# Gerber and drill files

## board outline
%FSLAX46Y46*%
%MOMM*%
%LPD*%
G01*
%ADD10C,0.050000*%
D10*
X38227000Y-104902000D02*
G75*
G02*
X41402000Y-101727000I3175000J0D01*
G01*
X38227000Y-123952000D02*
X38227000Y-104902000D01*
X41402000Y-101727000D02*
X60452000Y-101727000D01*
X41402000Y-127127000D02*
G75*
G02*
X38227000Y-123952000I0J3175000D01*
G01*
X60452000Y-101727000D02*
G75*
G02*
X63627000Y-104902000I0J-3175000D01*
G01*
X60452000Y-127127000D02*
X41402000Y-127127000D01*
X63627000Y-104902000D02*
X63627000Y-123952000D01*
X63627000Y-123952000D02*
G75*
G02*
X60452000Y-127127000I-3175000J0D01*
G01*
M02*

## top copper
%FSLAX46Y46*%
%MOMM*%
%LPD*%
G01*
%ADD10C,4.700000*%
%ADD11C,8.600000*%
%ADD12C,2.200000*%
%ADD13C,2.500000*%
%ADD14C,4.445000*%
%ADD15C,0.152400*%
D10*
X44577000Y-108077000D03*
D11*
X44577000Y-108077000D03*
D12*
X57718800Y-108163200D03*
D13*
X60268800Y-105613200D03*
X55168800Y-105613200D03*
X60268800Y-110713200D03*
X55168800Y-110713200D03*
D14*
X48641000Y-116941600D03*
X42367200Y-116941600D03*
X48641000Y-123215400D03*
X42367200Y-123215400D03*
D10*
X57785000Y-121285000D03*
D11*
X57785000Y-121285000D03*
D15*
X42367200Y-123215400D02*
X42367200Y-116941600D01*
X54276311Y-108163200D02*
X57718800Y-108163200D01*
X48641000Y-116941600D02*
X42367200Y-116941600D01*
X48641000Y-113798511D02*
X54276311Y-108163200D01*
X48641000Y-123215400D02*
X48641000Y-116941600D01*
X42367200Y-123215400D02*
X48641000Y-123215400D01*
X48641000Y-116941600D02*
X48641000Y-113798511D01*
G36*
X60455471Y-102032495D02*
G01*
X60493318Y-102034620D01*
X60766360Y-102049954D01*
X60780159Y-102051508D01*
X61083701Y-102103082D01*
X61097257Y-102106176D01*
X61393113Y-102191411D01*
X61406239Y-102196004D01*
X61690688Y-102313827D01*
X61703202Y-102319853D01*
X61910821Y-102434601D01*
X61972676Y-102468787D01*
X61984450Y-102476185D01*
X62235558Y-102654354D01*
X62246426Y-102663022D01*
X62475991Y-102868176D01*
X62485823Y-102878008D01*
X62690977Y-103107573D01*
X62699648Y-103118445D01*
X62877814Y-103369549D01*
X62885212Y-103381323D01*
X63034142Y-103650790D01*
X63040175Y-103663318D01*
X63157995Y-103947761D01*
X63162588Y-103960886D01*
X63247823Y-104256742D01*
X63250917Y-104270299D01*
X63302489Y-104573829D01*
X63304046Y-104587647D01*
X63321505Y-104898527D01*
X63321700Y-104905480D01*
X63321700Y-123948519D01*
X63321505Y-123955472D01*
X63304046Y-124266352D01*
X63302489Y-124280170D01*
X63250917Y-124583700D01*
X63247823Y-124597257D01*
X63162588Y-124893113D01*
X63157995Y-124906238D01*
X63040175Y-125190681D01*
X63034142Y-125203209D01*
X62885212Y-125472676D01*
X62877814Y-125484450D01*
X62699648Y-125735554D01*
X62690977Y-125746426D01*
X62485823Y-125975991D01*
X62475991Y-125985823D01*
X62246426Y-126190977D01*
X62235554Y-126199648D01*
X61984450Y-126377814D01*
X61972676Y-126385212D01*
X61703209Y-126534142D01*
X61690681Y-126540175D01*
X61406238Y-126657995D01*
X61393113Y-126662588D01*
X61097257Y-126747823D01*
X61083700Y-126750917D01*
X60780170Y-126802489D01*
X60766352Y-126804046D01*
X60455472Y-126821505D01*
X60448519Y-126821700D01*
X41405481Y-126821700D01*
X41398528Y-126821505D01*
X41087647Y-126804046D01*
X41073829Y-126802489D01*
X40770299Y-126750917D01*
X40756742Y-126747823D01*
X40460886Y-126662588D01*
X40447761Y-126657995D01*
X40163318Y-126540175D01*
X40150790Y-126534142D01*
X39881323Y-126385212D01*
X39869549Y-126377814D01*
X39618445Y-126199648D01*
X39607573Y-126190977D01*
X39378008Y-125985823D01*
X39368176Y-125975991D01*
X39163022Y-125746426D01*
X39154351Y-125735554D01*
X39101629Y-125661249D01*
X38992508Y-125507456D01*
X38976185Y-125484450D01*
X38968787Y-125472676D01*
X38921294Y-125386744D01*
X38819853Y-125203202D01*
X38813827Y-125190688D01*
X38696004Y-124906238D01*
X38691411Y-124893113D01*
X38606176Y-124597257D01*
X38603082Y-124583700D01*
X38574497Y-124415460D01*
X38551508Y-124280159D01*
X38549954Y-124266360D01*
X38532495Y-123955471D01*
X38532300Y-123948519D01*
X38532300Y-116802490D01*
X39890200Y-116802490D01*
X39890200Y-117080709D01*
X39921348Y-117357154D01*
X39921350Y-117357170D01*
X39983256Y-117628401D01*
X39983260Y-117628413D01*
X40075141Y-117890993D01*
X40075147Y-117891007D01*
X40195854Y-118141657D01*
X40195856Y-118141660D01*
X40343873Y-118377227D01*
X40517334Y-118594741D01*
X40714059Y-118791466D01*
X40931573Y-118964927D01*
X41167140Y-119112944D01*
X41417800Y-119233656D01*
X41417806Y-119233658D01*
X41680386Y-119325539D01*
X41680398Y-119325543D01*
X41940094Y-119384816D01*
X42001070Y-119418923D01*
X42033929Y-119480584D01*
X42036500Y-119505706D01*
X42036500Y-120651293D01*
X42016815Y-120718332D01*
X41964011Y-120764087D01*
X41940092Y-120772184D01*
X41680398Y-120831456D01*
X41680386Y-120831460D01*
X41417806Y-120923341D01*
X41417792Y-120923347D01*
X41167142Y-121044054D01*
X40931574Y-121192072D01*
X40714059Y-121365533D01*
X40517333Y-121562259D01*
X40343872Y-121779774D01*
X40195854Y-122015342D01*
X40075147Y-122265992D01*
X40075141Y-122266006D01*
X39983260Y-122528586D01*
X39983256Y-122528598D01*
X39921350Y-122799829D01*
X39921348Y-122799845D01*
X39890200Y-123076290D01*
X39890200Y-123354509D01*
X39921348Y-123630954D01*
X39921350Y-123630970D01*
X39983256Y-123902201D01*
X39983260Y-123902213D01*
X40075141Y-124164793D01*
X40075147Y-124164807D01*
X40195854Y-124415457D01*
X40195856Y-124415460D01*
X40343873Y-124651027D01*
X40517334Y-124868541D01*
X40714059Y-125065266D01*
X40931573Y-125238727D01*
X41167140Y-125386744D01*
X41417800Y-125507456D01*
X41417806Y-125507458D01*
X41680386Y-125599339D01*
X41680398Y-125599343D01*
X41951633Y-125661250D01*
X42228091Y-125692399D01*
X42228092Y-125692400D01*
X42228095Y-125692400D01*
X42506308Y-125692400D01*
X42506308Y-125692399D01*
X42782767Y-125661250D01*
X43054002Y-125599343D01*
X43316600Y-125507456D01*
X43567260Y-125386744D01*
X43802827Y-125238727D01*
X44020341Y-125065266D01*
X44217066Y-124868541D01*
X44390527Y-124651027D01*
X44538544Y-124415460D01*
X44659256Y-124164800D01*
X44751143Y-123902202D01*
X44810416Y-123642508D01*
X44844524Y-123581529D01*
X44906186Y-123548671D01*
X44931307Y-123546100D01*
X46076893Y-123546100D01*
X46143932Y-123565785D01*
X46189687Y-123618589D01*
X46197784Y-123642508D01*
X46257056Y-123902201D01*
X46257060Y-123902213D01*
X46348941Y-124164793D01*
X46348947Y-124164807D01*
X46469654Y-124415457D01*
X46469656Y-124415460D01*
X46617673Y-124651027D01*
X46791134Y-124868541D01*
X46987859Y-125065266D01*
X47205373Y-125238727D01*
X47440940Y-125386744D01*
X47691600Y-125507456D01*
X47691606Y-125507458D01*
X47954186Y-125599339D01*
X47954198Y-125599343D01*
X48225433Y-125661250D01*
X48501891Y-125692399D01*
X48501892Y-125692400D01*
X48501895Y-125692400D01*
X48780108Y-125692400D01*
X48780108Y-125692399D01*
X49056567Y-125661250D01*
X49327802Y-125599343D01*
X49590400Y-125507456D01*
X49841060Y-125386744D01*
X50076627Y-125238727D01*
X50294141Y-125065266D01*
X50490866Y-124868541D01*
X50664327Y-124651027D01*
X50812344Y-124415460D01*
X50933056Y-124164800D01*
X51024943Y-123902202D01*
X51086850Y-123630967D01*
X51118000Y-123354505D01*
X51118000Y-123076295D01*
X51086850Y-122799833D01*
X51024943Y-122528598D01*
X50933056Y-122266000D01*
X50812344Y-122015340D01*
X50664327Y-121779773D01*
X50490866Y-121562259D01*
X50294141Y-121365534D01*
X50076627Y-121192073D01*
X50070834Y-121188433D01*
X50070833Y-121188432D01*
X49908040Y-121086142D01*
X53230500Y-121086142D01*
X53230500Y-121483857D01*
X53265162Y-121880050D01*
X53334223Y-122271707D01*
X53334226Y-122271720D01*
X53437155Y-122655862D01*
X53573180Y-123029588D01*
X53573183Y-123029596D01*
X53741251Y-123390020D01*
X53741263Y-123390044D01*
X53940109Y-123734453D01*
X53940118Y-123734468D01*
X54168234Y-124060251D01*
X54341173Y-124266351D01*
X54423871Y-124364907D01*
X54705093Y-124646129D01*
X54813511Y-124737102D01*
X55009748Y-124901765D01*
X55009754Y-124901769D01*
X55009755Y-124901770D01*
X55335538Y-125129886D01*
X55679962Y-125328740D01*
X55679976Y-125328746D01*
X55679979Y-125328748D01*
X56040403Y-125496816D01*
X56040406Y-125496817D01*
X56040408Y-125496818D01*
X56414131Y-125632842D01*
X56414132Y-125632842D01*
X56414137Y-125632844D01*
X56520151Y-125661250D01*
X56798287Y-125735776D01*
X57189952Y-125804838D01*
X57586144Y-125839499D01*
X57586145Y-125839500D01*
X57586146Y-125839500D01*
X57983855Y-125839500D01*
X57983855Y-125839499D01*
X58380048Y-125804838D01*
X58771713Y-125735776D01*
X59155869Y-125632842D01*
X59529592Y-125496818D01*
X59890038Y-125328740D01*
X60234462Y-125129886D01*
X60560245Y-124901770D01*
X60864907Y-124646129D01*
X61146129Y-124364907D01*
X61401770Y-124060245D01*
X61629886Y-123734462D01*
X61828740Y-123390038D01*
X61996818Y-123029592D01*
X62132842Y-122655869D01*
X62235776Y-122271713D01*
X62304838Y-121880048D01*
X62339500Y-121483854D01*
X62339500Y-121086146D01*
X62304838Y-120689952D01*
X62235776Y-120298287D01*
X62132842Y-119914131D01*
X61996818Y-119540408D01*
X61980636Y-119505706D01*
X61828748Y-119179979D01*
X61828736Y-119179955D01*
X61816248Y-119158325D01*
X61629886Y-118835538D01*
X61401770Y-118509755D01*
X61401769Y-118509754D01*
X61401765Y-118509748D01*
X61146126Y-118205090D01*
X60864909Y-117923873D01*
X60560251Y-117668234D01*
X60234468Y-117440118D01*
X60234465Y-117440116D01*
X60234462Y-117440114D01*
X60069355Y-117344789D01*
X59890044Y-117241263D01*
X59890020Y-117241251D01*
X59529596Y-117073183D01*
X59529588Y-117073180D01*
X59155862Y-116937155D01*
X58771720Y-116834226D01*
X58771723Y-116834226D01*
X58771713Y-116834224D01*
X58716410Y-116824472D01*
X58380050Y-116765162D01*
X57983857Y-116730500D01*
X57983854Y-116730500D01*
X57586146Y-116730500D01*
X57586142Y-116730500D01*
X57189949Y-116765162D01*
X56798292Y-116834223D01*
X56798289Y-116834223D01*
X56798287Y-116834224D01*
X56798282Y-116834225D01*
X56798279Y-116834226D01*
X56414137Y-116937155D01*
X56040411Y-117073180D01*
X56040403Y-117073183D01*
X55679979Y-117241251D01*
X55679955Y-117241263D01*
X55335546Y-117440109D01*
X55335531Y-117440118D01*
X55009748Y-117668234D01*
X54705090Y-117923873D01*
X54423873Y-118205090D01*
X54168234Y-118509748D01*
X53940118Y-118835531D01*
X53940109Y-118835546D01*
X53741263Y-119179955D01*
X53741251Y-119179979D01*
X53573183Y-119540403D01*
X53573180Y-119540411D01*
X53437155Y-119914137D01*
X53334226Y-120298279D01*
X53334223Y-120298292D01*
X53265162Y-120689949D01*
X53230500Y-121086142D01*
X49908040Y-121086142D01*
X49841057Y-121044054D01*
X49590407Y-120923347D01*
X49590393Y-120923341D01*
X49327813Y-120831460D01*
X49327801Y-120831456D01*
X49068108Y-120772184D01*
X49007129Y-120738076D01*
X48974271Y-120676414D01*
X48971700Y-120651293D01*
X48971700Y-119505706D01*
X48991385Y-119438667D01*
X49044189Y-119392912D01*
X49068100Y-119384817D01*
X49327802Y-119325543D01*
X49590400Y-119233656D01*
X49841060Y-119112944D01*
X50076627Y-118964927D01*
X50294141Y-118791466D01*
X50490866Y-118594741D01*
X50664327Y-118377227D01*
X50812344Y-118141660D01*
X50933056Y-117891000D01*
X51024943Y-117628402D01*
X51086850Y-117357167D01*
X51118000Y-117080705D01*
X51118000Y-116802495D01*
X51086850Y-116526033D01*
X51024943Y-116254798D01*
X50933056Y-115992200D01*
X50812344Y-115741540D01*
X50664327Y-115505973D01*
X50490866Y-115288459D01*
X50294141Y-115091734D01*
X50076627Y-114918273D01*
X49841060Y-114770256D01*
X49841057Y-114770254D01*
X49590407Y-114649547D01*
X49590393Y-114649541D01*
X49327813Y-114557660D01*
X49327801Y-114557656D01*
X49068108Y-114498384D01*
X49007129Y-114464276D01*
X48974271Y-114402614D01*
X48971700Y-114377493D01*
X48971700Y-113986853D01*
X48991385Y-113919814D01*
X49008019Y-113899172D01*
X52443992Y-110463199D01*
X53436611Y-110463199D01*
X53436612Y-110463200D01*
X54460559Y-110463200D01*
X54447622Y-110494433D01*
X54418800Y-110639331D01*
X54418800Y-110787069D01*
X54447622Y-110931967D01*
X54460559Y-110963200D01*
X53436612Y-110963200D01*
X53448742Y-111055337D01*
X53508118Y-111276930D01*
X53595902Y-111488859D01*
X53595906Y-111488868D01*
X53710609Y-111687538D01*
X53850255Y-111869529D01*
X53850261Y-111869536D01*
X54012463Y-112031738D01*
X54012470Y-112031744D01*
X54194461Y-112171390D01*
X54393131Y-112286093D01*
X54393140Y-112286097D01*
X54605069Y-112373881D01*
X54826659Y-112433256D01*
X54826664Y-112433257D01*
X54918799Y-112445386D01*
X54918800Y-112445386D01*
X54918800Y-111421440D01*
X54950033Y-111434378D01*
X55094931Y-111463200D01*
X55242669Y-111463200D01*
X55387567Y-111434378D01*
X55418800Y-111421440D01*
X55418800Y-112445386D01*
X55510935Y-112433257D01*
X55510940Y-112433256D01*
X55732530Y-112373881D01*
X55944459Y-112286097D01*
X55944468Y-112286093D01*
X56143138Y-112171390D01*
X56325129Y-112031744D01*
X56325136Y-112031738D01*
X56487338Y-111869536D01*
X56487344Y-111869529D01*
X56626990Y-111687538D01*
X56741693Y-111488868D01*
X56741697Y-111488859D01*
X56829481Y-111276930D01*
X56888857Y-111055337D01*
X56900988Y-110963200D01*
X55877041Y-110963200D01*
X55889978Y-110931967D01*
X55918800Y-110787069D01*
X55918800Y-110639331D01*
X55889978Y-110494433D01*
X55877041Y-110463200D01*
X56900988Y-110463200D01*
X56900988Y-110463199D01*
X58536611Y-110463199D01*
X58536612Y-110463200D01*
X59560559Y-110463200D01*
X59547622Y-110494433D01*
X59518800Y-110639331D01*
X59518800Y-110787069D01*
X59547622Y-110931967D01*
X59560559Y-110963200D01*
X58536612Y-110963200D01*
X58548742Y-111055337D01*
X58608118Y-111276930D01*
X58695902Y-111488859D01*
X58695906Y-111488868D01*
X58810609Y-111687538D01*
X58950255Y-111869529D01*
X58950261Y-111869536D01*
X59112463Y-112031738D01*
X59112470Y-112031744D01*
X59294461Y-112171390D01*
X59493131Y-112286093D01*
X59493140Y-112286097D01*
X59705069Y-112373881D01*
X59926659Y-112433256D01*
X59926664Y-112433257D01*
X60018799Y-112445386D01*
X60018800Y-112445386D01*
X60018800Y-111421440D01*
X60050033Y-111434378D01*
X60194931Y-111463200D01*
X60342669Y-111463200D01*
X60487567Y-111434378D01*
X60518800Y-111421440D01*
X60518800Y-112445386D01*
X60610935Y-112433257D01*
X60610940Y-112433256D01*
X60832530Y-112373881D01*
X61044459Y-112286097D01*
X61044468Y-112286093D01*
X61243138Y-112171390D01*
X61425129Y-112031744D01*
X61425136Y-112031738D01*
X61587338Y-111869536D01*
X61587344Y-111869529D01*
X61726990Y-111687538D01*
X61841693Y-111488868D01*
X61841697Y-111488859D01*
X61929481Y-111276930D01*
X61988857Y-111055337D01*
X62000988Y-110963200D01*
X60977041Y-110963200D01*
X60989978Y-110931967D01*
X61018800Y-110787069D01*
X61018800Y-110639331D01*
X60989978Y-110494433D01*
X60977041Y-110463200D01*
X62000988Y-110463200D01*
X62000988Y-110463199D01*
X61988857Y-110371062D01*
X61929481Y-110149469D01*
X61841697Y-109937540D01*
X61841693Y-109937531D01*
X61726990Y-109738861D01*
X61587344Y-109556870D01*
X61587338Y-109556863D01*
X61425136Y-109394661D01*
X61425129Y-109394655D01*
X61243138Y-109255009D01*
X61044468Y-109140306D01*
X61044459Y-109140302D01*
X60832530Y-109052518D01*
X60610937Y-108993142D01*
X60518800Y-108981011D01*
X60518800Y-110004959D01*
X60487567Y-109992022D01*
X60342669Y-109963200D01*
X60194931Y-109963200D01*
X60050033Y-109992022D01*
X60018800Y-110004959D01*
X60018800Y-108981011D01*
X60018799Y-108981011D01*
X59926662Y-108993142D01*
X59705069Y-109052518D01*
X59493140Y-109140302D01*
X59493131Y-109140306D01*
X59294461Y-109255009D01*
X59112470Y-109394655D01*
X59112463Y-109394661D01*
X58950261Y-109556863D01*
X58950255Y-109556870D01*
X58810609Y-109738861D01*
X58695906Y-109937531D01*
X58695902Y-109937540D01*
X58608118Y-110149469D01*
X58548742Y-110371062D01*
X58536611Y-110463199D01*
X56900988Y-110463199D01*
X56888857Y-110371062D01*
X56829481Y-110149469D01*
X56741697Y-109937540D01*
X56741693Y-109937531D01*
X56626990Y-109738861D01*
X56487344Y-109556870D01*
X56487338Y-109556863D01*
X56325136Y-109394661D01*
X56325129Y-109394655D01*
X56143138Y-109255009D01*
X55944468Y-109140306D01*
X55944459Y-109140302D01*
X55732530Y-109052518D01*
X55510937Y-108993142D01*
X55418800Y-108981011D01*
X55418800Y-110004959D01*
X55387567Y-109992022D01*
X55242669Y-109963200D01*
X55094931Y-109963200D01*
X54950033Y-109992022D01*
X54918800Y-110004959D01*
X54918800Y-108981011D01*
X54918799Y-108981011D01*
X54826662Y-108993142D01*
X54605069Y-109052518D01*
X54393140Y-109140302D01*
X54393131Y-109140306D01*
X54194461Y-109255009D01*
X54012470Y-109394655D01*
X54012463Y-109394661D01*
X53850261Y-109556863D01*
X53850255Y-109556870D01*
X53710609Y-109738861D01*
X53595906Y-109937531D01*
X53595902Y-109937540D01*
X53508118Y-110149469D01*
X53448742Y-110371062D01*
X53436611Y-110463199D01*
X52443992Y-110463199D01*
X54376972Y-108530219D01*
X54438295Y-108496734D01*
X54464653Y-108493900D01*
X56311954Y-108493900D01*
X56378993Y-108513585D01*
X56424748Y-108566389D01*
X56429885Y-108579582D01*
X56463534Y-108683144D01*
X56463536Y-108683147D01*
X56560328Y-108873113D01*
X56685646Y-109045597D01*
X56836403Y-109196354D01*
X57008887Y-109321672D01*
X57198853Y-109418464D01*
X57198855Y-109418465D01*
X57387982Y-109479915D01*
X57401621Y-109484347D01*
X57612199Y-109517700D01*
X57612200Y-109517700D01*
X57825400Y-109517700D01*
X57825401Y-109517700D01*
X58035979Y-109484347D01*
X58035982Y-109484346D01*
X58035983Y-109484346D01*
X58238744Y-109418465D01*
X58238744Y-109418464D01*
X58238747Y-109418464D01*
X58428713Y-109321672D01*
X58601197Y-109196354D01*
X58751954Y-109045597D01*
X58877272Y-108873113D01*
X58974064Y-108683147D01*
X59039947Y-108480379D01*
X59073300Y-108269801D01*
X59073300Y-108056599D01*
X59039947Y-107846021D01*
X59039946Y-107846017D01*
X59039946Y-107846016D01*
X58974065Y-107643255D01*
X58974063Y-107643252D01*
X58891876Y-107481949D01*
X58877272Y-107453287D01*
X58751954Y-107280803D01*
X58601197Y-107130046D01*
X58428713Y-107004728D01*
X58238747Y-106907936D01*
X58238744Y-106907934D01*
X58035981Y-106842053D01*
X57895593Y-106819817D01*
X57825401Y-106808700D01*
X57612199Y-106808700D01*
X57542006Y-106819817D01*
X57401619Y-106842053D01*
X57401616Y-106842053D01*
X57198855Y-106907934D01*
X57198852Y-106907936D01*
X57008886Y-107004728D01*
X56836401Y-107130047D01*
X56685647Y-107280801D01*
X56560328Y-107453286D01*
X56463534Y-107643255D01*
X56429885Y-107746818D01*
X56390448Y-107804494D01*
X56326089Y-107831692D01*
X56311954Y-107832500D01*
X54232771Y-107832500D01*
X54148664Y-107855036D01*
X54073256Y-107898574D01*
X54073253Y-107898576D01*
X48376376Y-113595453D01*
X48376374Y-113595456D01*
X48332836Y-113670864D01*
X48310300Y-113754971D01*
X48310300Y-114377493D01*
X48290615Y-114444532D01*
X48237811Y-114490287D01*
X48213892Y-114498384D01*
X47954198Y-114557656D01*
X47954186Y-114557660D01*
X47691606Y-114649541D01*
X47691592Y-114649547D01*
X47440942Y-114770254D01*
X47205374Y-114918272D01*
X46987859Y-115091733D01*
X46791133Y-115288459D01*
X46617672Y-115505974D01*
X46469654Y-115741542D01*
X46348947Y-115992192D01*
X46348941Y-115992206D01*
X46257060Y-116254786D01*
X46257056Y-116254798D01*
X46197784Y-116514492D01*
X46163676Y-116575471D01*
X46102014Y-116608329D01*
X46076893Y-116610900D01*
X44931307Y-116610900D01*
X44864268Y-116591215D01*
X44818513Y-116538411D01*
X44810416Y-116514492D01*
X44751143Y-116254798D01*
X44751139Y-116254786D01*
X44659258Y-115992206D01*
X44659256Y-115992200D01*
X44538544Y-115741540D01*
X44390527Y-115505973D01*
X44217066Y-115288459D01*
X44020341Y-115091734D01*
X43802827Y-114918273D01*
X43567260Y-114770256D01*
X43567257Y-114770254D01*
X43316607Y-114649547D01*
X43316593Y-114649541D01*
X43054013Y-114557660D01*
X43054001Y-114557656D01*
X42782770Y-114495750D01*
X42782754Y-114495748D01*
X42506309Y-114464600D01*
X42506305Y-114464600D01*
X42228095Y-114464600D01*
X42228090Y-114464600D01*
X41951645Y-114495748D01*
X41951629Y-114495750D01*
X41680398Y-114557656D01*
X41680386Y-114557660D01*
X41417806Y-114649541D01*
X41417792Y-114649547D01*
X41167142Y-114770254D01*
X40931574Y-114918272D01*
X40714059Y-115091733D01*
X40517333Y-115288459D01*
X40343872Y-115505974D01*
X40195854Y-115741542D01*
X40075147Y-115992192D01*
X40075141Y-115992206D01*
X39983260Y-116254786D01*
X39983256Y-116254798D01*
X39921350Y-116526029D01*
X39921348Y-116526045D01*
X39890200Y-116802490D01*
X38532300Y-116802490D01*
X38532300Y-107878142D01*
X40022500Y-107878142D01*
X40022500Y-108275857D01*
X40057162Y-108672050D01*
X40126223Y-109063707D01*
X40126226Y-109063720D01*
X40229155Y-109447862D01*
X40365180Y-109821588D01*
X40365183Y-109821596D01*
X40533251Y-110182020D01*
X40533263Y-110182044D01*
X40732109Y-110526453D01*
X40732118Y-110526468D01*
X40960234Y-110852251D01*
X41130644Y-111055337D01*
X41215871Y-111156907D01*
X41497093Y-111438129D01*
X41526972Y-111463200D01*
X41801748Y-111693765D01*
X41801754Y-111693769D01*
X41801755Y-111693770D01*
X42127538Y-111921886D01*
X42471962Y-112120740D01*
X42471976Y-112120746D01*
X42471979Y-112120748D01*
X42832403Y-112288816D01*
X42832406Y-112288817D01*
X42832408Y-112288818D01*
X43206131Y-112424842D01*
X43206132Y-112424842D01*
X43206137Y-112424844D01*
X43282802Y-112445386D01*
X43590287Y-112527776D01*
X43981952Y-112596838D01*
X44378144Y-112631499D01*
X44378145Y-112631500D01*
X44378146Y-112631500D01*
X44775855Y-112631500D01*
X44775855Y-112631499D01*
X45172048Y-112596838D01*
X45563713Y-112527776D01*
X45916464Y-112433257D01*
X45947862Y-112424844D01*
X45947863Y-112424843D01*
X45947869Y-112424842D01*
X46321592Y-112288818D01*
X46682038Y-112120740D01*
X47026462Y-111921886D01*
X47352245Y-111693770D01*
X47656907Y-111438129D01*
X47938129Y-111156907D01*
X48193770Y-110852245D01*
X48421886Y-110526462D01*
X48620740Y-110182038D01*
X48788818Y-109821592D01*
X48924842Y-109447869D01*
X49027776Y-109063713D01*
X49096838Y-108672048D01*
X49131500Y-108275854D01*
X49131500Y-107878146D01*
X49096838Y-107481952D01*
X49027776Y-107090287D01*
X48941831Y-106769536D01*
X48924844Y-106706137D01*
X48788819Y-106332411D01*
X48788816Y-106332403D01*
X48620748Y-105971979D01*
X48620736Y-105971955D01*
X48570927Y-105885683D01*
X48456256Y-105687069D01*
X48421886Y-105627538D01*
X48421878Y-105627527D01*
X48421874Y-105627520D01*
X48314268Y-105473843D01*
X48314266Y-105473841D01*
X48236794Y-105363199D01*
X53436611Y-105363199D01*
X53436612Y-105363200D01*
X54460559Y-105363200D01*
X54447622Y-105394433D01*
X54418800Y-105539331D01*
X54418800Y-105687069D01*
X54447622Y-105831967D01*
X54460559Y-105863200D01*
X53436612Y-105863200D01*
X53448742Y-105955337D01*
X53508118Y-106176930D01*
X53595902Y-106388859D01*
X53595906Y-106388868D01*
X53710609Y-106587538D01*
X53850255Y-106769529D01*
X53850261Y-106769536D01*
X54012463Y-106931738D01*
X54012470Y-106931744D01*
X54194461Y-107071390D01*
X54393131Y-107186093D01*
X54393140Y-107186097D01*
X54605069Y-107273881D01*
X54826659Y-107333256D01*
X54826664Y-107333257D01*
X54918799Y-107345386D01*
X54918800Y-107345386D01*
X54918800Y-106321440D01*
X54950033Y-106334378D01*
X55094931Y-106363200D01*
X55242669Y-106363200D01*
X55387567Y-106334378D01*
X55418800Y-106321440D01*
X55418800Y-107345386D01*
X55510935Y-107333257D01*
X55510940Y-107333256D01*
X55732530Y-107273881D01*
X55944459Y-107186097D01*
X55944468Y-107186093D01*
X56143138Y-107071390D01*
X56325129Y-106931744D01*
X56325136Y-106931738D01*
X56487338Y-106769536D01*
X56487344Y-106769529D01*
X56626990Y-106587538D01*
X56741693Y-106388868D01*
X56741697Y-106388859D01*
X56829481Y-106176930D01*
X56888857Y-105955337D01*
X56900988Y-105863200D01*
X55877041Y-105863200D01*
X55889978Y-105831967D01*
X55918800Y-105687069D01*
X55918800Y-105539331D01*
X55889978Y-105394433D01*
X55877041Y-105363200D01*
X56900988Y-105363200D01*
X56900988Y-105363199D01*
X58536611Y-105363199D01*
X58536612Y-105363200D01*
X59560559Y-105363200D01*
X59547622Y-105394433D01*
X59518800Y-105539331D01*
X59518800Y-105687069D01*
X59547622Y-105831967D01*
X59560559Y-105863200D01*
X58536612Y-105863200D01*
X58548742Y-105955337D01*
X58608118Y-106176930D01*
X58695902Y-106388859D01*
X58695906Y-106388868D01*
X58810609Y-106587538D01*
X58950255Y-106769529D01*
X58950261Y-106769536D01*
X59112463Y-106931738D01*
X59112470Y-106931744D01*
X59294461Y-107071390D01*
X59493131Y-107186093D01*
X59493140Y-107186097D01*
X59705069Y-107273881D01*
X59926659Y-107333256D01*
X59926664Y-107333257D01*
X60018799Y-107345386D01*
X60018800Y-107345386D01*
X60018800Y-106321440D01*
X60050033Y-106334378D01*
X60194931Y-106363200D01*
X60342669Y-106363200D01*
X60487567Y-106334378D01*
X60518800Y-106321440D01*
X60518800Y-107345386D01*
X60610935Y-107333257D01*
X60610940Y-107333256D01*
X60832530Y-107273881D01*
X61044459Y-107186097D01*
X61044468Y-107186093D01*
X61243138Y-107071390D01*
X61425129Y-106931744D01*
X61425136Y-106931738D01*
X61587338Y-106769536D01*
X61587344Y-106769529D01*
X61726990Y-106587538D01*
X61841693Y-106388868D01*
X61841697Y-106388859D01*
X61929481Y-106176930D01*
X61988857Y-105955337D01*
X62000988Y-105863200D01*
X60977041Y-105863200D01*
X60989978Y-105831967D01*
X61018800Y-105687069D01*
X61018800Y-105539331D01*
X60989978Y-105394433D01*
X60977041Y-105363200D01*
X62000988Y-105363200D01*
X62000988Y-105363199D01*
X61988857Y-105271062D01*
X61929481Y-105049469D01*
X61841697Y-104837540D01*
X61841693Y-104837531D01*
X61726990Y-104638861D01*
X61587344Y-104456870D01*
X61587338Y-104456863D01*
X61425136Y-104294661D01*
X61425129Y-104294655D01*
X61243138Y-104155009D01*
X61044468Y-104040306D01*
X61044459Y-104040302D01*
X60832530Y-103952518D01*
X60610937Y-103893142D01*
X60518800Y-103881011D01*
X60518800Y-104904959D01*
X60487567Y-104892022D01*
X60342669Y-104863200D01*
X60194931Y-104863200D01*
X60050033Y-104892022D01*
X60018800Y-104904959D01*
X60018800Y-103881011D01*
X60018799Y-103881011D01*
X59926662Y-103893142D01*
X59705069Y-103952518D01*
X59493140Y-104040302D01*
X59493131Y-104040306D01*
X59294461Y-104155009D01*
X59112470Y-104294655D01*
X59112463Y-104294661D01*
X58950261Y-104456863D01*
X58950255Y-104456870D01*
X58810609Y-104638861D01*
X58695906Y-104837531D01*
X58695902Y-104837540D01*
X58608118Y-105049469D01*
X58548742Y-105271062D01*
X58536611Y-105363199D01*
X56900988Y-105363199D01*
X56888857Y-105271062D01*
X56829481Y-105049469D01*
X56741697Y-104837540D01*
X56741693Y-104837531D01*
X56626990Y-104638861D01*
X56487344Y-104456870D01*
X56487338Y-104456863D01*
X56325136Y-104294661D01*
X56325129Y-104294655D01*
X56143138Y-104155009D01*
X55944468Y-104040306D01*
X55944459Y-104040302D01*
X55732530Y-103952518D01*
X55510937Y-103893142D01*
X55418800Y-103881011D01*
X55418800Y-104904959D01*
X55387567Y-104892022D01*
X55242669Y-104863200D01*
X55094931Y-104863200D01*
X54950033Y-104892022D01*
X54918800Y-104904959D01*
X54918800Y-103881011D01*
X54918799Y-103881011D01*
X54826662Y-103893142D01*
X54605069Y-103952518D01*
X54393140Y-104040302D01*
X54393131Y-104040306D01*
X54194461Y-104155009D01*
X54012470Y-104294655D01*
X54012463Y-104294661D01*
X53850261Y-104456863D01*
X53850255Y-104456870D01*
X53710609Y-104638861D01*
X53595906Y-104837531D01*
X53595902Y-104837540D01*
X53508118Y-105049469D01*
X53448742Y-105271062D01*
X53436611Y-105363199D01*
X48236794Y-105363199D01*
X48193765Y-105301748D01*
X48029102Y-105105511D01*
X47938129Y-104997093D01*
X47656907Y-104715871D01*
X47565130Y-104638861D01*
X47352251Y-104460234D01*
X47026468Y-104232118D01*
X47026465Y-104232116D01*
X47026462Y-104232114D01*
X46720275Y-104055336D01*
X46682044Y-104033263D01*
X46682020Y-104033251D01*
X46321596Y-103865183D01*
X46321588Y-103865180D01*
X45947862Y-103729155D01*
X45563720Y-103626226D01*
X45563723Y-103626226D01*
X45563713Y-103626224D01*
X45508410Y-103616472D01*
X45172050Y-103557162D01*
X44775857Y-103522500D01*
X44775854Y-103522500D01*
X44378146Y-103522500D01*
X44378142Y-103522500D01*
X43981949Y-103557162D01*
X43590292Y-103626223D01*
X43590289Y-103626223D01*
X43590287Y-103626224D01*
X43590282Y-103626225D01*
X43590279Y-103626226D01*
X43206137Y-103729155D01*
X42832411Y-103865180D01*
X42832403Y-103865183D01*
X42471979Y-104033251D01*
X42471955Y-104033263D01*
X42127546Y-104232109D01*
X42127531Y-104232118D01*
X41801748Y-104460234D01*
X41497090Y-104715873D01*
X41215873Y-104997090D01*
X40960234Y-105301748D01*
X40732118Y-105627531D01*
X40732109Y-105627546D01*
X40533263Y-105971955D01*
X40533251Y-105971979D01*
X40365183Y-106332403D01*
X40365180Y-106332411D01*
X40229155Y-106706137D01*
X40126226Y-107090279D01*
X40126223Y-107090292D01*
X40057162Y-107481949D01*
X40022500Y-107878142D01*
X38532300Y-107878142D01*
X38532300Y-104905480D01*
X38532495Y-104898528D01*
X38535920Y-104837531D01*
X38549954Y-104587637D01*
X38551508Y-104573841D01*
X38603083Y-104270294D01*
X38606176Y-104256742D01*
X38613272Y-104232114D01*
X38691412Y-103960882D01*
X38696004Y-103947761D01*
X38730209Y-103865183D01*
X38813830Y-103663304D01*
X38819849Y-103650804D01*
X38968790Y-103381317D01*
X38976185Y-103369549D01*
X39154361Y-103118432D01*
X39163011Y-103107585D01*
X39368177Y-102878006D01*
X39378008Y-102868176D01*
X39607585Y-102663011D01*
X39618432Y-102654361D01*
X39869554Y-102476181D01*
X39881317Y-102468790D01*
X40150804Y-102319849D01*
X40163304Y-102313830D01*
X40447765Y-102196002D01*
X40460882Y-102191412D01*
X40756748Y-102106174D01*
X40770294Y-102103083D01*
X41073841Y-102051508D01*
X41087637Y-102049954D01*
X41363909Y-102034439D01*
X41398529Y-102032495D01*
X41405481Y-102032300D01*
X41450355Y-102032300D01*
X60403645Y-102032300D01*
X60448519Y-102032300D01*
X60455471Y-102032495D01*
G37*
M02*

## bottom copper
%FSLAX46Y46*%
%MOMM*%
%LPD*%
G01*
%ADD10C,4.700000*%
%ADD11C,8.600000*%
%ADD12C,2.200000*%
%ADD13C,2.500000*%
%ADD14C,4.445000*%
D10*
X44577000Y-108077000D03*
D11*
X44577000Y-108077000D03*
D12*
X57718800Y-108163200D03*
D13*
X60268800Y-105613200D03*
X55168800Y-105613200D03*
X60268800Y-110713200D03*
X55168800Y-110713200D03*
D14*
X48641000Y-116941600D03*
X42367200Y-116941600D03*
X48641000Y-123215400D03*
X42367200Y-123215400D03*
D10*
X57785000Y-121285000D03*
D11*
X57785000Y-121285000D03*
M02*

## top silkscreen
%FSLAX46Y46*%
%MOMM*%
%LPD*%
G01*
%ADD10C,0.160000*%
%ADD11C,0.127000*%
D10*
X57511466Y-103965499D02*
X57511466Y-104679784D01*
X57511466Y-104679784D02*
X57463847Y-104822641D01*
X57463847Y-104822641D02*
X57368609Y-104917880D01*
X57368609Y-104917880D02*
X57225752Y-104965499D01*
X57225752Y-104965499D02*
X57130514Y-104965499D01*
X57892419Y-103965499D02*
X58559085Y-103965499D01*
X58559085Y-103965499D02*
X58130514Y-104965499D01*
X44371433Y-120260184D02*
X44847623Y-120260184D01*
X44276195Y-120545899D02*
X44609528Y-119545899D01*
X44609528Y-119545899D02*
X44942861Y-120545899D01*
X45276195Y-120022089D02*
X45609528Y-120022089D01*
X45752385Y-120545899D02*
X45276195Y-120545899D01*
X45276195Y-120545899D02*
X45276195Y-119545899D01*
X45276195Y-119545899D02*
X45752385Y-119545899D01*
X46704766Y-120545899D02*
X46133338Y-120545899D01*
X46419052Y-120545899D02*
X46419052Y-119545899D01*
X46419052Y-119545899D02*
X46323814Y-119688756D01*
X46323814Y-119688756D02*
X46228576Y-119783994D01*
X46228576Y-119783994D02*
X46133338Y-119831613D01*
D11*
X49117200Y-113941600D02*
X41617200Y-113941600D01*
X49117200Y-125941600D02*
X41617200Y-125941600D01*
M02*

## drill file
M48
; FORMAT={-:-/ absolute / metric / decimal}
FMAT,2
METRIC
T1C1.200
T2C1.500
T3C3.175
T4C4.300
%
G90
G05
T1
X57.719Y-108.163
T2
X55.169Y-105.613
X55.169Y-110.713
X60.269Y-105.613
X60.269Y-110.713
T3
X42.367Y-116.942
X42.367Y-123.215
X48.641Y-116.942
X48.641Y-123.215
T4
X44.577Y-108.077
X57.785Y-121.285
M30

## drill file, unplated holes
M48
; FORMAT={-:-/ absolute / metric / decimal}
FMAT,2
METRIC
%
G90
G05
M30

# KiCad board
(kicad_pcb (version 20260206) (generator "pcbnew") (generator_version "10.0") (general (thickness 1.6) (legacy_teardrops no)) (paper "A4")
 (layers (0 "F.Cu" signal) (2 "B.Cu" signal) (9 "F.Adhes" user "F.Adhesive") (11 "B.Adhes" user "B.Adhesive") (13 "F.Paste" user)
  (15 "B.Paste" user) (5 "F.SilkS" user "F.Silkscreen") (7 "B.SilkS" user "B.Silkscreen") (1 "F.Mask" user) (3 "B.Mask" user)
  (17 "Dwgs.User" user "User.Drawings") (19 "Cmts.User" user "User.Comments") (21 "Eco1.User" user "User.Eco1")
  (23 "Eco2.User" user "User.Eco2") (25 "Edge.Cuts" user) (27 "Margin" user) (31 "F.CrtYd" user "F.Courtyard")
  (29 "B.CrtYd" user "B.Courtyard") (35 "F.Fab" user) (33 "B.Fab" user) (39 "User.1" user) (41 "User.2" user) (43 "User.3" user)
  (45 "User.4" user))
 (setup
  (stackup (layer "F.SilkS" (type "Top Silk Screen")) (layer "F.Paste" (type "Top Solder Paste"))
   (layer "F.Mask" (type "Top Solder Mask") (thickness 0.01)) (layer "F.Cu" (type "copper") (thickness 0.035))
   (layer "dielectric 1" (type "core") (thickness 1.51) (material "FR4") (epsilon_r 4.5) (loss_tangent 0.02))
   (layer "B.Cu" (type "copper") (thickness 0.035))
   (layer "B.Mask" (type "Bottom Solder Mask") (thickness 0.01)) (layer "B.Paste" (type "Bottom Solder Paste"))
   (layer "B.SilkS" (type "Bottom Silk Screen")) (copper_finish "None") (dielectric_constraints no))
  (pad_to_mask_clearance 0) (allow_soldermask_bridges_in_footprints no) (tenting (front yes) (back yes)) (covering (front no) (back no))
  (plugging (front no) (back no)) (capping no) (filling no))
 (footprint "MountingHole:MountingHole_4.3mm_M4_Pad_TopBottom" (layer "F.Cu") (at 44.577 108.077)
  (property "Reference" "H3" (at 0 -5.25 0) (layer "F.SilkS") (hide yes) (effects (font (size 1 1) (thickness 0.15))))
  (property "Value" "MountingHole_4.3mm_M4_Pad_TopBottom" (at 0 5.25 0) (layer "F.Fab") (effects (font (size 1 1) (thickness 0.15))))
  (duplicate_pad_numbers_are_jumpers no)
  (pad "1" thru_hole circle (at 0 0) (size 4.7 4.7) (drill 4.3) (layers "*.Cu" "*.Mask") (remove_unused_layers no) (zone_connect 2))
  (pad "1" connect circle (at 0 0) (size 8.6 8.6) (layers "F.Cu" "F.Mask") (zone_connect 2))
  (pad "1" connect circle (at 0 0) (size 8.6 8.6) (layers "B.Cu" "B.Mask") (zone_connect 2)))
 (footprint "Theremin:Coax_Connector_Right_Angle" (layer "F.Cu") (at 55.1688 105.6132 -90)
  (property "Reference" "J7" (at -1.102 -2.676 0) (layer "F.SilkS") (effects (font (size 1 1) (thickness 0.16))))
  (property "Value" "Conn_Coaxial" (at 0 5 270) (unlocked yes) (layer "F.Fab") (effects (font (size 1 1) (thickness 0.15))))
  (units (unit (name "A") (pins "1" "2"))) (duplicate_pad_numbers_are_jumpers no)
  (pad "1" thru_hole circle (at 2.55 -2.55 270) (size 2.2 2.2) (drill 1.2) (layers "*.Cu" "*.Mask") (remove_unused_layers no)
   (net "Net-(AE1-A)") (thermal_bridge_angle 90))
  (pad "2" thru_hole circle (at 0 -5.1 270) (size 2.5 2.5) (drill 1.5) (layers "*.Cu" "*.Mask") (remove_unused_layers no) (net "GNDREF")
   (thermal_bridge_angle 90))
  (pad "2" thru_hole circle (at 0 0 270) (size 2.5 2.5) (drill 1.5) (layers "*.Cu" "*.Mask") (remove_unused_layers no) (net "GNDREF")
   (thermal_bridge_angle 90))
  (pad "2" thru_hole circle (at 5.1 -5.1 270) (size 2.5 2.5) (drill 1.5) (layers "*.Cu" "*.Mask") (remove_unused_layers no) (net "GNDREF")
   (thermal_bridge_angle 90))
  (pad "2" thru_hole circle (at 5.1 0 270) (size 2.5 2.5) (drill 1.5) (layers "*.Cu" "*.Mask") (remove_unused_layers no) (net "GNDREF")
   (thermal_bridge_angle 90)))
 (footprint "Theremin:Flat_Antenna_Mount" (layer "F.Cu") (at 42.3672 116.9416 -90)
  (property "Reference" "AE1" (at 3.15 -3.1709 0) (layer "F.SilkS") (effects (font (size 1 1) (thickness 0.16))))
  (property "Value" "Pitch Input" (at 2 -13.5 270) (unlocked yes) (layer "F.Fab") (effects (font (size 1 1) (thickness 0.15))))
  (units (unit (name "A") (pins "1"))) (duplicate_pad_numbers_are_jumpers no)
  (fp_line (start -3 -6.75) (end -3 0.75) (stroke (width 0.127) (type default)) (layer "F.SilkS"))
  (fp_line (start 9 -6.75) (end 9 0.75) (stroke (width 0.127) (type default)) (layer "F.SilkS"))
  (pad "1" thru_hole circle (at 0 -6.2738 270) (size 4.445 4.445) (drill 3.175) (layers "*.Cu" "*.Mask") (remove_unused_layers no)
   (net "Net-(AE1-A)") (thermal_bridge_angle 90))
  (pad "1" thru_hole circle (at 0 0 270) (size 4.445 4.445) (drill 3.175) (layers "*.Cu" "*.Mask") (remove_unused_layers no)
   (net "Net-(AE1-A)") (thermal_bridge_angle 90))
  (pad "1" thru_hole circle (at 6.2738 -6.2738 270) (size 4.445 4.445) (drill 3.175) (layers "*.Cu" "*.Mask") (remove_unused_layers no)
   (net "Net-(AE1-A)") (thermal_bridge_angle 90))
  (pad "1" thru_hole circle (at 6.2738 0 270) (size 4.445 4.445) (drill 3.175) (layers "*.Cu" "*.Mask") (remove_unused_layers no)
   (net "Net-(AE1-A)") (thermal_bridge_angle 90)))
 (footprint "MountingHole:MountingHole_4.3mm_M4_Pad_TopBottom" (layer "F.Cu") (at 57.785 121.285)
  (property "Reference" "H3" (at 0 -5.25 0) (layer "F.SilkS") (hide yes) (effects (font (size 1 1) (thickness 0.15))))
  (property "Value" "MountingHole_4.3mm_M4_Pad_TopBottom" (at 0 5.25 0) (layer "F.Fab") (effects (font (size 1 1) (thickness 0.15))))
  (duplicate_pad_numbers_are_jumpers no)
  (pad "1" thru_hole circle (at 0 0) (size 4.7 4.7) (drill 4.3) (layers "*.Cu" "*.Mask") (remove_unused_layers no) (zone_connect 2))
  (pad "1" connect circle (at 0 0) (size 8.6 8.6) (layers "F.Cu" "F.Mask") (zone_connect 2))
  (pad "1" connect circle (at 0 0) (size 8.6 8.6) (layers "B.Cu" "B.Mask") (zone_connect 2)))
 (gr_arc (start 38.227 104.902) (mid 39.156936 102.656936) (end 41.402 101.727) (stroke (width 0.05) (type default)) (layer "Edge.Cuts"))
 (gr_line (start 38.227 123.952) (end 38.227 104.902) (stroke (width 0.05) (type default)) (layer "Edge.Cuts"))
 (gr_line (start 41.402 101.727) (end 60.452 101.727) (stroke (width 0.05) (type default)) (layer "Edge.Cuts"))
 (gr_arc (start 41.402 127.127) (mid 39.156936 126.197064) (end 38.227 123.952) (stroke (width 0.05) (type default)) (layer "Edge.Cuts"))
 (gr_arc (start 60.452 101.727) (mid 62.697064 102.656936) (end 63.627 104.902) (stroke (width 0.05) (type default)) (layer "Edge.Cuts"))
 (gr_line (start 60.452 127.127) (end 41.402 127.127) (stroke (width 0.05) (type default)) (layer "Edge.Cuts"))
 (gr_line (start 63.627 104.902) (end 63.627 123.952) (stroke (width 0.05) (type default)) (layer "Edge.Cuts"))
 (gr_arc (start 63.627 123.952) (mid 62.697064 126.197064) (end 60.452 127.127) (stroke (width 0.05) (type default)) (layer "Edge.Cuts"))
 (segment (start 42.3672 123.2154) (end 42.3672 116.9416) (width 0.1524) (layer "F.Cu") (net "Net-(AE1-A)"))
 (segment (start 54.276311 108.1632) (end 57.7188 108.1632) (width 0.1524) (layer "F.Cu") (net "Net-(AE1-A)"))
 (segment (start 48.641 116.9416) (end 42.3672 116.9416) (width 0.1524) (layer "F.Cu") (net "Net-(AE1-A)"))
 (segment (start 48.641 113.798511) (end 54.276311 108.1632) (width 0.1524) (layer "F.Cu") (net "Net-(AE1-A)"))
 (segment (start 48.641 123.2154) (end 48.641 116.9416) (width 0.1524) (layer "F.Cu") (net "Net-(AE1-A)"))
 (segment (start 42.3672 123.2154) (end 48.641 123.2154) (width 0.1524) (layer "F.Cu") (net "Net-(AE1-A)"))
 (segment (start 48.641 116.9416) (end 48.641 113.798511) (width 0.1524) (layer "F.Cu") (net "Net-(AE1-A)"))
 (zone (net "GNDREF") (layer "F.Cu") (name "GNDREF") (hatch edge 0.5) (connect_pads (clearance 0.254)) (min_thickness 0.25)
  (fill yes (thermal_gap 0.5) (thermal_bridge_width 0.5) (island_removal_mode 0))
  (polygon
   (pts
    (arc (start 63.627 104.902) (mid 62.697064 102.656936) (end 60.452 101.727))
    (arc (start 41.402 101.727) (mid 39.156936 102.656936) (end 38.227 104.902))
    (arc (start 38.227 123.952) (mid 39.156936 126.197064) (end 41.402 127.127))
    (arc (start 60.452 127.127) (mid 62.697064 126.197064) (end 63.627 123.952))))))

